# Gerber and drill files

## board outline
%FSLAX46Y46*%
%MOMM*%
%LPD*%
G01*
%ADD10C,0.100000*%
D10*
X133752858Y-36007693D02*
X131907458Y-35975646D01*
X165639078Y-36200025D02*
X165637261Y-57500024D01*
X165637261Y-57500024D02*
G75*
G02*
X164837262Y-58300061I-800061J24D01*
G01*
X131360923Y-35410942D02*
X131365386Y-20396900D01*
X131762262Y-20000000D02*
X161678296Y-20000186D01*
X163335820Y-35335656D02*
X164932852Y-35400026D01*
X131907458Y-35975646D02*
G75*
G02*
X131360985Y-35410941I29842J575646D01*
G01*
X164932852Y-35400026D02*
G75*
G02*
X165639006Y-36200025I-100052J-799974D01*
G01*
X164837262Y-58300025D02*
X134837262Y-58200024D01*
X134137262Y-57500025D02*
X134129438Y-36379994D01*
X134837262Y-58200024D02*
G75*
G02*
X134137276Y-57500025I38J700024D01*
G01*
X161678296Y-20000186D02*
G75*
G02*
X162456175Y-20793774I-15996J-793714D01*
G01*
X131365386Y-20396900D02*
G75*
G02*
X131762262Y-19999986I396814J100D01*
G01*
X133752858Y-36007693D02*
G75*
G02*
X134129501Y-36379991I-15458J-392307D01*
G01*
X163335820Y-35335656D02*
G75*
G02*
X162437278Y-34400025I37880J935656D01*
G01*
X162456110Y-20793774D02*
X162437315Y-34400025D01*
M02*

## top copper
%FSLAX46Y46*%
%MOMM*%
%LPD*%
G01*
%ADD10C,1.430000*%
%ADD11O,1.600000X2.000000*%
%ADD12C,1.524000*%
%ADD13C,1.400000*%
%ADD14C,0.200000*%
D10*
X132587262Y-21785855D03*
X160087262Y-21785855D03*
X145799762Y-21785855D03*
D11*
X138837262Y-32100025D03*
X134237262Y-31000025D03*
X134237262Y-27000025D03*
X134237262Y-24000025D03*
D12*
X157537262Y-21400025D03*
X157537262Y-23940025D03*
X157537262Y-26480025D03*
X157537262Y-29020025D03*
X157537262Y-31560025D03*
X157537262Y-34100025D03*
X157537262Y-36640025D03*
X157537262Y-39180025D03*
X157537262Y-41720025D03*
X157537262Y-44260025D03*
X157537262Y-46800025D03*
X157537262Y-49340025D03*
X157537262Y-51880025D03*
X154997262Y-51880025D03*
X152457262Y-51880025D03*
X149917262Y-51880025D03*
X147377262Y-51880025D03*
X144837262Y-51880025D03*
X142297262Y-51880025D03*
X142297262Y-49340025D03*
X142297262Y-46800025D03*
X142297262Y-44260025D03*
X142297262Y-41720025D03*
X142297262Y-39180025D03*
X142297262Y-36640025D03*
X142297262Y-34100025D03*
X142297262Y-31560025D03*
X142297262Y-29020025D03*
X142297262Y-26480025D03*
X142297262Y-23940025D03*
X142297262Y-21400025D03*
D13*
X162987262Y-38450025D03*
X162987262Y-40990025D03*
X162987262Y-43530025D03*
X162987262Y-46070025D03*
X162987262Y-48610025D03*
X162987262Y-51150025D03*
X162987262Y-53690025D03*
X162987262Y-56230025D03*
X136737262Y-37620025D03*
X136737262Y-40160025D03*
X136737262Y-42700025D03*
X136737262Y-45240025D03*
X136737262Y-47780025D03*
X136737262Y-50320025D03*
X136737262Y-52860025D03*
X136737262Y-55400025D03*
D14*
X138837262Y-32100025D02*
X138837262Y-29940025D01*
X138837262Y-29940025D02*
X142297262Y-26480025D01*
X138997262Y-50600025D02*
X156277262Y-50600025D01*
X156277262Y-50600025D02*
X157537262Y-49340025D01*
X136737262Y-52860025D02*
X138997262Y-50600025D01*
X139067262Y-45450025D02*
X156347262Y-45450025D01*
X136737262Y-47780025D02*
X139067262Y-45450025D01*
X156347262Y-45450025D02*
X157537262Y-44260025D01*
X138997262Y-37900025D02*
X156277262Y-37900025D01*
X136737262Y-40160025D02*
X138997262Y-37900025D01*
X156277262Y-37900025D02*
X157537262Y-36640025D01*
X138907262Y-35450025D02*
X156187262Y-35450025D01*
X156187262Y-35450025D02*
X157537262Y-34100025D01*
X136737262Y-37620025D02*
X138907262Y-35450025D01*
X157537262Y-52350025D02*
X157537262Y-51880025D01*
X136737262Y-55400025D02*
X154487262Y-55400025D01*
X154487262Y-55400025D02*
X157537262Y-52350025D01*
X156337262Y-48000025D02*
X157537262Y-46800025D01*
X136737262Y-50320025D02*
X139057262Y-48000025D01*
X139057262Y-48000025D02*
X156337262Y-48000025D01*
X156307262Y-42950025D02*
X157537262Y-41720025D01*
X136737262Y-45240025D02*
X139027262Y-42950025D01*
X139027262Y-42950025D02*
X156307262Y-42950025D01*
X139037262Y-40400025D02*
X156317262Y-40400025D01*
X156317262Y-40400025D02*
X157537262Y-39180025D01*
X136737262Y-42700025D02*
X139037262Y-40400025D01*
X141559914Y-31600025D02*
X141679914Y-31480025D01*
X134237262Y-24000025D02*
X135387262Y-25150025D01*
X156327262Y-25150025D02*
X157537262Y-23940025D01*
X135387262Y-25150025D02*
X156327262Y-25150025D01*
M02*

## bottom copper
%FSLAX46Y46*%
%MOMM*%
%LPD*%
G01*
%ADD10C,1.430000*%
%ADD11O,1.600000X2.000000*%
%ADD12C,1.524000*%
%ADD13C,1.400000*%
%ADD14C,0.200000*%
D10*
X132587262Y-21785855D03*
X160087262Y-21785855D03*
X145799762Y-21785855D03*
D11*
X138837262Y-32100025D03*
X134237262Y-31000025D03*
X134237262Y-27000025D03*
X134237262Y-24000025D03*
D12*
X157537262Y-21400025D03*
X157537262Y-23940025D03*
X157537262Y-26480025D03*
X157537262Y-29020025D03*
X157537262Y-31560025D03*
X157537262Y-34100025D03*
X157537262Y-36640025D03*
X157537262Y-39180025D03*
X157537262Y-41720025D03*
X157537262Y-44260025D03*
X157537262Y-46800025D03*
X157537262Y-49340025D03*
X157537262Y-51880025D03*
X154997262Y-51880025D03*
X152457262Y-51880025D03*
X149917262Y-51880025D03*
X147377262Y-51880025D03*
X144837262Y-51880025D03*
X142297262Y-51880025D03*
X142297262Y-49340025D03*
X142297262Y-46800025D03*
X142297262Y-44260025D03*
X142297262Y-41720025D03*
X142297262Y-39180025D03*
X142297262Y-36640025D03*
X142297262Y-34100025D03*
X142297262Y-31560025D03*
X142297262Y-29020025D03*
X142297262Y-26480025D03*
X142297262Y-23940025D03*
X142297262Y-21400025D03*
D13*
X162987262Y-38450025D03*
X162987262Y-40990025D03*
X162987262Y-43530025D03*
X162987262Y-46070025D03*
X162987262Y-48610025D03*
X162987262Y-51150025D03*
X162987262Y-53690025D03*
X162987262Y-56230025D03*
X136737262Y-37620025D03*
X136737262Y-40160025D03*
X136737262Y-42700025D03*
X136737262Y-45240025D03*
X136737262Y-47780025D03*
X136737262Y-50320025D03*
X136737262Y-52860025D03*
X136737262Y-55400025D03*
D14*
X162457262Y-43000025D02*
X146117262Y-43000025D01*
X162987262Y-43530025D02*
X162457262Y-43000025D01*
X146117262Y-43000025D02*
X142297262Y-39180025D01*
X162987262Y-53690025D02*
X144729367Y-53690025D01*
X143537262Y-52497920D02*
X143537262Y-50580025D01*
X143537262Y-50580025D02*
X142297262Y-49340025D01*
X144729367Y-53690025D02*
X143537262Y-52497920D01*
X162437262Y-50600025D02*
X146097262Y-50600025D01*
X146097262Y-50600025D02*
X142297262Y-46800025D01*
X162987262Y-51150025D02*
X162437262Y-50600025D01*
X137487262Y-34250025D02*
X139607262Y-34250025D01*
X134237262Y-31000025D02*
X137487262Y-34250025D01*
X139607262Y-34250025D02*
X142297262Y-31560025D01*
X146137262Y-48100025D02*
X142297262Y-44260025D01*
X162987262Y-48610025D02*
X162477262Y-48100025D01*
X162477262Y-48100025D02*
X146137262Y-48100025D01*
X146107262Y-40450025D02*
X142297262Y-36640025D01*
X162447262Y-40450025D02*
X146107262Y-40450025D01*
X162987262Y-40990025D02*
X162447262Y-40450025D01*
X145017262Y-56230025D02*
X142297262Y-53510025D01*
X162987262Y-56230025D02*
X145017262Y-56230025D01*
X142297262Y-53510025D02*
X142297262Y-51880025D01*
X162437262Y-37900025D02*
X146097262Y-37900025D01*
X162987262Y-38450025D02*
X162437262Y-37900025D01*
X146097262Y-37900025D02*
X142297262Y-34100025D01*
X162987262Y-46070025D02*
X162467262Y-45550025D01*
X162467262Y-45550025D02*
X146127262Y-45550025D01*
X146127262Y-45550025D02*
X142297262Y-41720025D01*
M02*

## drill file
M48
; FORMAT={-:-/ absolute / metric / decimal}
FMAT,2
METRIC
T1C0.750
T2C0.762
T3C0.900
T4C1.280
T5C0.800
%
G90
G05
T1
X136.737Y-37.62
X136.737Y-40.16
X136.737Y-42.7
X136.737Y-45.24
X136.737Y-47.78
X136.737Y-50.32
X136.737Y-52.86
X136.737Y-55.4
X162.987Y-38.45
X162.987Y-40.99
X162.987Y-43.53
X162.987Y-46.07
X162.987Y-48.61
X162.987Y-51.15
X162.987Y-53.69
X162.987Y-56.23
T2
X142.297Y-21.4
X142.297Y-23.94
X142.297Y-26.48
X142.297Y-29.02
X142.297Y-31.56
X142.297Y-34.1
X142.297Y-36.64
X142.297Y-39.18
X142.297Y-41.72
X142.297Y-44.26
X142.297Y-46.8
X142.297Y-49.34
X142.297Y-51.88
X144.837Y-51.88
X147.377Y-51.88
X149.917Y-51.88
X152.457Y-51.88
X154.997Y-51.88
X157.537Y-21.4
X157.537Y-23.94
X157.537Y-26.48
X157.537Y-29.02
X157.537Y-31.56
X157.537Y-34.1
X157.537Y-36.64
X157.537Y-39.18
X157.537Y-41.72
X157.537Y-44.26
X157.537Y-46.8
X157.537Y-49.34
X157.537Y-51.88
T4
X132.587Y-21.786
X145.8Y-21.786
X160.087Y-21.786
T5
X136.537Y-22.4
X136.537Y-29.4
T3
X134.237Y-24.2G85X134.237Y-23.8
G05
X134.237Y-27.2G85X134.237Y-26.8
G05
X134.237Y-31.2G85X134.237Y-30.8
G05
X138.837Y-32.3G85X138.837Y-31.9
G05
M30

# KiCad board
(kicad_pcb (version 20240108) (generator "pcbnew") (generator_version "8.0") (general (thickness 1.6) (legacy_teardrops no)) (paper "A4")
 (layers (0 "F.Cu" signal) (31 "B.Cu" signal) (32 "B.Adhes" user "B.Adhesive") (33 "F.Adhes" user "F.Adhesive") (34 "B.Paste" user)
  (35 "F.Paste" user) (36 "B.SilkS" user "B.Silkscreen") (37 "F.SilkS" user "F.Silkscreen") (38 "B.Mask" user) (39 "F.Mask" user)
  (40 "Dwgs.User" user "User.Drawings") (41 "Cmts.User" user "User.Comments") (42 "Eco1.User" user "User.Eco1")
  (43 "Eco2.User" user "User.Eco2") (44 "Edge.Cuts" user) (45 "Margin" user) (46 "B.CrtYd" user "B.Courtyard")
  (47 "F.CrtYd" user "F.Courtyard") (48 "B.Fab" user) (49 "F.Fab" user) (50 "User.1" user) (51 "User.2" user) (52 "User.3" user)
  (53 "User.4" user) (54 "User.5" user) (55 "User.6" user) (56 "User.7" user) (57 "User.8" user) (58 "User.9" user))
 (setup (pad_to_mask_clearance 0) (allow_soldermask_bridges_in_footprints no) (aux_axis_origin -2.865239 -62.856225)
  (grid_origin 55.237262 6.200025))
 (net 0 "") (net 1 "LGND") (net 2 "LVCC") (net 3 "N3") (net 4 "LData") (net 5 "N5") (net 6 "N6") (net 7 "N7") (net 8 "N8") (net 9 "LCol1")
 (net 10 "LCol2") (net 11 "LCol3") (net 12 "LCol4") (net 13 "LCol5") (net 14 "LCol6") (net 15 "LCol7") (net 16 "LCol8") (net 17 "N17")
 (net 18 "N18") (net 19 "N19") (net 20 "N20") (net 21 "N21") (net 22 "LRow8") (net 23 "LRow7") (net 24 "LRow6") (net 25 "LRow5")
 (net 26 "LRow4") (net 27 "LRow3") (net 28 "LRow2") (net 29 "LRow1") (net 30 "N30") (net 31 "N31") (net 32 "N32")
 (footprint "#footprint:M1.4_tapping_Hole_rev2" (layer "F.Cu") (at 148.137262 23.700025 -90)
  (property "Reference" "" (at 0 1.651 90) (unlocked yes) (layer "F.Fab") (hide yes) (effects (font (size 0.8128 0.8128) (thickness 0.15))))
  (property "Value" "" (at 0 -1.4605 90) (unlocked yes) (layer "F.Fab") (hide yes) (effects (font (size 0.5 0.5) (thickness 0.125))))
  (pad "" thru_hole circle (at -1.91417 15.55 270) (size 1.43 1.43) (drill 1.28) (layers "*.Cu" "*.Mask") (remove_unused_layers no)))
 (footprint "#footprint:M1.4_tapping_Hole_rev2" (layer "F.Cu") (at 160.087262 21.785855 -90)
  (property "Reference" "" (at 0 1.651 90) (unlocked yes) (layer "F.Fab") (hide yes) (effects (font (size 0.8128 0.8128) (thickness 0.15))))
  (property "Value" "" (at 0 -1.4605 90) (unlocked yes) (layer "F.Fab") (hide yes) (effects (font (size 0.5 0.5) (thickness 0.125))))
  (pad "" thru_hole circle (at 0 0 270) (size 1.43 1.43) (drill 1.28) (layers "*.Cu" "*.Mask") (remove_unused_layers no)))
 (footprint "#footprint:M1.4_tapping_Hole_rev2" (layer "F.Cu") (at 145.799762 21.785855 -90)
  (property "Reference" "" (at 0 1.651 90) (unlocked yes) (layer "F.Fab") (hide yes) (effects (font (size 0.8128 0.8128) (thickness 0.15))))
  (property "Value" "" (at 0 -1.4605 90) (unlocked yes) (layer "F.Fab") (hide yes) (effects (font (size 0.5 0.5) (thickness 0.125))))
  (pad "" thru_hole circle (at 0 0 270) (size 1.43 1.43) (drill 1.28) (layers "*.Cu" "*.Mask") (remove_unused_layers no)))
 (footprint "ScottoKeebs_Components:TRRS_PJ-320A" (layer "B.Cu") (at 136.537262 20.800025 180)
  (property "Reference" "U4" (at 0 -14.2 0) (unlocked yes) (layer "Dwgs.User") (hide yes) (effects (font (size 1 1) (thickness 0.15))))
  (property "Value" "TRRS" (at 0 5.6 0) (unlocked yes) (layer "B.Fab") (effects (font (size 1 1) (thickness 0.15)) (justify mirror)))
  (pad "" np_thru_hole circle (at 0 -8.6 180) (size 0.8 0.8) (drill 0.8) (layers "*.Cu" "*.Mask"))
  (pad "" np_thru_hole circle (at 0 -1.6 180) (size 0.8 0.8) (drill 0.8) (layers "*.Cu" "*.Mask"))
  (pad "1" thru_hole oval (at -2.3 -11.3 180) (size 1.6 2) (drill oval 0.9 1.3) (layers "*.Cu" "*.Mask") (remove_unused_layers no)
   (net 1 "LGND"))
  (pad "2" thru_hole oval (at 2.3 -10.2 180) (size 1.6 2) (drill oval 0.9 1.3) (layers "*.Cu" "*.Mask") (remove_unused_layers no)
   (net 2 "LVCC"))
  (pad "3" thru_hole oval (at 2.3 -6.2 180) (size 1.6 2) (drill oval 0.9 1.3) (layers "*.Cu" "*.Mask") (remove_unused_layers no)
   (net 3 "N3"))
  (pad "4" thru_hole oval (at 2.3 -3.2 180) (size 1.6 2) (drill oval 0.9 1.3) (layers "*.Cu" "*.Mask") (remove_unused_layers no)
   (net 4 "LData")))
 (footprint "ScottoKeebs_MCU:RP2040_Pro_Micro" (layer "B.Cu") (at 149.917262 37.910025 180)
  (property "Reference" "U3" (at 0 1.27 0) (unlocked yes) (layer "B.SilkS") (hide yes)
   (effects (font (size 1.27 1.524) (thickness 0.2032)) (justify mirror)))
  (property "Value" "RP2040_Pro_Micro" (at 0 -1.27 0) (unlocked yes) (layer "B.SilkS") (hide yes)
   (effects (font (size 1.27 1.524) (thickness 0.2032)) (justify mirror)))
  (pad "1" thru_hole circle (at -7.62 16.51 180) (size 1.524 1.524) (drill 0.762) (layers "*.Cu" "*.Mask") (remove_unused_layers no)
   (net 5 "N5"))
  (pad "2" thru_hole circle (at -7.62 13.97 180) (size 1.524 1.524) (drill 0.762) (layers "*.Cu" "*.Mask") (remove_unused_layers no)
   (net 4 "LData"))
  (pad "3" thru_hole circle (at -7.62 11.43 180) (size 1.524 1.524) (drill 0.762) (layers "*.Cu" "*.Mask") (remove_unused_layers no)
   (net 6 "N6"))
  (pad "4" thru_hole circle (at -7.62 8.89 180) (size 1.524 1.524) (drill 0.762) (layers "*.Cu" "*.Mask") (remove_unused_layers no)
   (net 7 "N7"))
  (pad "5" thru_hole circle (at -7.62 6.35 180) (size 1.524 1.524) (drill 0.762) (layers "*.Cu" "*.Mask") (remove_unused_layers no)
   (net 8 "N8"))
  (pad "6" thru_hole circle (at -7.62 3.81 180) (size 1.524 1.524) (drill 0.762) (layers "*.Cu" "*.Mask") (remove_unused_layers no)
   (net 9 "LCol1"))
  (pad "7" thru_hole circle (at -7.62 1.27 180) (size 1.524 1.524) (drill 0.762) (layers "*.Cu" "*.Mask") (remove_unused_layers no)
   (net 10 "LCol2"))
  (pad "8" thru_hole circle (at -7.62 -1.27 180) (size 1.524 1.524) (drill 0.762) (layers "*.Cu" "*.Mask") (remove_unused_layers no)
   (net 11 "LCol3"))
  (pad "9" thru_hole circle (at -7.62 -3.81 180) (size 1.524 1.524) (drill 0.762) (layers "*.Cu" "*.Mask") (remove_unused_layers no)
   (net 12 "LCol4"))
  (pad "10" thru_hole circle (at -7.62 -6.35 180) (size 1.524 1.524) (drill 0.762) (layers "*.Cu" "*.Mask") (remove_unused_layers no)
   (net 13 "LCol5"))
  (pad "11" thru_hole circle (at -7.62 -8.89 180) (size 1.524 1.524) (drill 0.762) (layers "*.Cu" "*.Mask") (remove_unused_layers no)
   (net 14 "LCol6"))
  (pad "12" thru_hole circle (at -7.62 -11.43 180) (size 1.524 1.524) (drill 0.762) (layers "*.Cu" "*.Mask") (remove_unused_layers no)
   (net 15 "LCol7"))
  (pad "13" thru_hole circle (at -7.62 -13.97 180) (size 1.524 1.524) (drill 0.762) (layers "*.Cu" "*.Mask") (remove_unused_layers no)
   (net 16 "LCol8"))
  (pad "14" thru_hole circle (at -5.08 -13.97 180) (size 1.524 1.524) (drill 0.762) (layers "*.Cu" "*.Mask") (remove_unused_layers no)
   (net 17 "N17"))
  (pad "15" thru_hole circle (at -2.54 -13.97 180) (size 1.524 1.524) (drill 0.762) (layers "*.Cu" "*.Mask") (remove_unused_layers no)
   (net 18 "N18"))
  (pad "16" thru_hole circle (at 0 -13.97 180) (size 1.524 1.524) (drill 0.762) (layers "*.Cu" "*.Mask") (remove_unused_layers no)
   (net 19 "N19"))
  (pad "17" thru_hole circle (at 2.54 -13.97 180) (size 1.524 1.524) (drill 0.762) (layers "*.Cu" "*.Mask") (remove_unused_layers no)
   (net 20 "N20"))
  (pad "18" thru_hole circle (at 5.08 -13.97 180) (size 1.524 1.524) (drill 0.762) (layers "*.Cu" "*.Mask") (remove_unused_layers no)
   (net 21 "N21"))
  (pad "19" thru_hole circle (at 7.62 -13.97 180) (size 1.524 1.524) (drill 0.762) (layers "*.Cu" "*.Mask") (remove_unused_layers no)
   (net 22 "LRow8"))
  (pad "20" thru_hole circle (at 7.62 -11.43 180) (size 1.524 1.524) (drill 0.762) (layers "*.Cu" "*.Mask") (remove_unused_layers no)
   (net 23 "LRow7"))
  (pad "21" thru_hole circle (at 7.62 -8.89 180) (size 1.524 1.524) (drill 0.762) (layers "*.Cu" "*.Mask") (remove_unused_layers no)
   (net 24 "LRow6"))
  (pad "22" thru_hole circle (at 7.62 -6.35 180) (size 1.524 1.524) (drill 0.762) (layers "*.Cu" "*.Mask") (remove_unused_layers no)
   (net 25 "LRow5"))
  (pad "23" thru_hole circle (at 7.62 -3.81 180) (size 1.524 1.524) (drill 0.762) (layers "*.Cu" "*.Mask") (remove_unused_layers no)
   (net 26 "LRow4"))
  (pad "24" thru_hole circle (at 7.62 -1.27 180) (size 1.524 1.524) (drill 0.762) (layers "*.Cu" "*.Mask") (remove_unused_layers no)
   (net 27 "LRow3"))
  (pad "25" thru_hole circle (at 7.62 1.27 180) (size 1.524 1.524) (drill 0.762) (layers "*.Cu" "*.Mask") (remove_unused_layers no)
   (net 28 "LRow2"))
  (pad "26" thru_hole circle (at 7.62 3.81 180) (size 1.524 1.524) (drill 0.762) (layers "*.Cu" "*.Mask") (remove_unused_layers no)
   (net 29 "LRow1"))
  (pad "27" thru_hole circle (at 7.62 6.35 180) (size 1.524 1.524) (drill 0.762) (layers "*.Cu" "*.Mask") (remove_unused_layers no)
   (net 2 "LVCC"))
  (pad "28" thru_hole circle (at 7.62 8.89 180) (size 1.524 1.524) (drill 0.762) (layers "*.Cu" "*.Mask") (remove_unused_layers no)
   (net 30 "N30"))
  (pad "29" thru_hole circle (at 7.62 11.43 180) (size 1.524 1.524) (drill 0.762) (layers "*.Cu" "*.Mask") (remove_unused_layers no)
   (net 1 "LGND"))
  (pad "30" thru_hole circle (at 7.62 13.97 180) (size 1.524 1.524) (drill 0.762) (layers "*.Cu" "*.Mask") (remove_unused_layers no)
   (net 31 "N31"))
  (pad "31" thru_hole circle (at 7.62 16.51 180) (size 1.524 1.524) (drill 0.762) (layers "*.Cu" "*.Mask") (remove_unused_layers no)
   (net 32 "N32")))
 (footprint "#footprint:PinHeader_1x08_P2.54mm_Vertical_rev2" (layer "B.Cu") (at 162.987262 38.450025 180)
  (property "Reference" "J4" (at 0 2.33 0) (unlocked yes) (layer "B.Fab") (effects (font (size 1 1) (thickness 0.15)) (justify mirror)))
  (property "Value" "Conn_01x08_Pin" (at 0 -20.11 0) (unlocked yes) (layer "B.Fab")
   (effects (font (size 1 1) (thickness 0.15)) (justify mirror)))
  (pad "1" thru_hole circle (at 0 0 180) (size 1.4 1.4) (drill 0.75) (layers "*.Cu" "*.Mask") (remove_unused_layers no) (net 29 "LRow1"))
  (pad "2" thru_hole circle (at 0 -2.54 180) (size 1.4 1.4) (drill 0.75) (layers "*.Cu" "*.Mask") (remove_unused_layers no) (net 28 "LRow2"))
  (pad "3" thru_hole circle (at 0 -5.08 180) (size 1.4 1.4) (drill 0.75) (layers "*.Cu" "*.Mask") (remove_unused_layers no) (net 27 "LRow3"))
  (pad "4" thru_hole circle (at 0 -7.62 180) (size 1.4 1.4) (drill 0.75) (layers "*.Cu" "*.Mask") (remove_unused_layers no) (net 26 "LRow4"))
  (pad "5" thru_hole circle (at 0 -10.16 180) (size 1.4 1.4) (drill 0.75) (layers "*.Cu" "*.Mask") (remove_unused_layers no)
   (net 25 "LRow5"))
  (pad "6" thru_hole circle (at 0 -12.7 180) (size 1.4 1.4) (drill 0.75) (layers "*.Cu" "*.Mask") (remove_unused_layers no) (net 24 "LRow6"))
  (pad "7" thru_hole circle (at 0 -15.24 180) (size 1.4 1.4) (drill 0.75) (layers "*.Cu" "*.Mask") (remove_unused_layers no)
   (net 23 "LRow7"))
  (pad "8" thru_hole circle (at 0 -17.78 180) (size 1.4 1.4) (drill 0.75) (layers "*.Cu" "*.Mask") (remove_unused_layers no)
   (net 22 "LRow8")))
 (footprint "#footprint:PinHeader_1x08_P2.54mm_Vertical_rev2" (layer "B.Cu") (at 136.737262 37.620025 180)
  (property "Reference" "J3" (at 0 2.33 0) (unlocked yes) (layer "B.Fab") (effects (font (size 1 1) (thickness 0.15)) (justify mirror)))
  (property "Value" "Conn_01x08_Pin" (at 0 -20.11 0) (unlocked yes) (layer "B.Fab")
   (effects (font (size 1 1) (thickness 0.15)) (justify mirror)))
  (pad "1" thru_hole circle (at 0 0 180) (size 1.4 1.4) (drill 0.75) (layers "*.Cu" "*.Mask") (remove_unused_layers no) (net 9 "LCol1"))
  (pad "2" thru_hole circle (at 0 -2.54 180) (size 1.4 1.4) (drill 0.75) (layers "*.Cu" "*.Mask") (remove_unused_layers no) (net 10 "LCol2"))
  (pad "3" thru_hole circle (at 0 -5.08 180) (size 1.4 1.4) (drill 0.75) (layers "*.Cu" "*.Mask") (remove_unused_layers no) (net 11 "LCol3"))
  (pad "4" thru_hole circle (at 0 -7.62 180) (size 1.4 1.4) (drill 0.75) (layers "*.Cu" "*.Mask") (remove_unused_layers no) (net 12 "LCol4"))
  (pad "5" thru_hole circle (at 0 -10.16 180) (size 1.4 1.4) (drill 0.75) (layers "*.Cu" "*.Mask") (remove_unused_layers no)
   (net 13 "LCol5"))
  (pad "6" thru_hole circle (at 0 -12.7 180) (size 1.4 1.4) (drill 0.75) (layers "*.Cu" "*.Mask") (remove_unused_layers no) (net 14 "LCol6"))
  (pad "7" thru_hole circle (at 0 -15.24 180) (size 1.4 1.4) (drill 0.75) (layers "*.Cu" "*.Mask") (remove_unused_layers no)
   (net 15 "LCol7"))
  (pad "8" thru_hole circle (at 0 -17.78 180) (size 1.4 1.4) (drill 0.75) (layers "*.Cu" "*.Mask") (remove_unused_layers no)
   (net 16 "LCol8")))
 (gr_line (start 133.752858 36.007693) (end 131.907458 35.975646) (stroke (width 0.1) (type default)) (layer "Edge.Cuts"))
 (gr_line (start 165.639078 36.200025) (end 165.637261 57.500024) (stroke (width 0.1) (type default)) (layer "Edge.Cuts"))
 (gr_arc (start 165.637261 57.500024) (mid 165.402937 58.0657) (end 164.837262 58.300025) (stroke (width 0.1) (type default))
  (layer "Edge.Cuts"))
 (gr_line (start 131.360923 35.410942) (end 131.365386 20.3969) (stroke (width 0.1) (type default)) (layer "Edge.Cuts"))
 (gr_line (start 131.762262 20) (end 161.678296 20.000186) (stroke (width 0.1) (type default)) (layer "Edge.Cuts"))
 (gr_line (start 163.33582 35.335656) (end 164.932852 35.400026) (stroke (width 0.1) (type default)) (layer "Edge.Cuts"))
 (gr_arc (start 131.907458 35.975646) (mid 131.523045 35.800863) (end 131.360923 35.410942) (stroke (width 0.1) (type default))
  (layer "Edge.Cuts"))
 (gr_arc (start 164.932852 35.400026) (mid 165.437261 35.666464) (end 165.639078 36.200025) (stroke (width 0.1) (type default))
  (layer "Edge.Cuts"))
 (gr_line (start 164.837262 58.300025) (end 134.837262 58.200024) (stroke (width 0.1) (type default)) (layer "Edge.Cuts"))
 (gr_line (start 134.137262 57.500025) (end 134.129438 36.379994) (stroke (width 0.1) (type default)) (layer "Edge.Cuts"))
 (gr_arc (start 134.837262 58.200024) (mid 134.342285 57.995001) (end 134.137262 57.500025) (stroke (width 0.1) (type default))
  (layer "Edge.Cuts"))
 (gr_arc (start 161.678296 20.000186) (mid 162.229203 20.2382) (end 162.45611 20.793774) (stroke (width 0.1) (type default))
  (layer "Edge.Cuts"))
 (gr_arc (start 131.365386 20.3969) (mid 131.481589 20.116221) (end 131.762262 20) (stroke (width 0.1) (type default)) (layer "Edge.Cuts"))
 (gr_arc (start 133.752858 36.007693) (mid 134.013376 36.120802) (end 134.129438 36.379994) (stroke (width 0.1) (type default))
  (layer "Edge.Cuts"))
 (gr_arc (start 163.33582 35.335656) (mid 162.698334 35.048622) (end 162.437315 34.400025) (stroke (width 0.1) (type default))
  (layer "Edge.Cuts"))
 (gr_line (start 162.45611 20.793774) (end 162.437315 34.400025) (stroke (width 0.1) (type default)) (layer "Edge.Cuts"))
 (segment (start 138.837262 32.100025) (end 138.837262 29.940025) (width 0.2) (layer "F.Cu") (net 1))
 (segment (start 138.837262 29.940025) (end 142.297262 26.480025) (width 0.2) (layer "F.Cu") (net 1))
 (segment (start 138.997262 50.600025) (end 156.277262 50.600025) (width 0.2) (layer "F.Cu") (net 15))
 (segment (start 156.277262 50.600025) (end 157.537262 49.340025) (width 0.2) (layer "F.Cu") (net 15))
 (segment (start 136.737262 52.860025) (end 138.997262 50.600025) (width 0.2) (layer "F.Cu") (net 15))
 (segment (start 139.067262 45.450025) (end 156.347262 45.450025) (width 0.2) (layer "F.Cu") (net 13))
 (segment (start 136.737262 47.780025) (end 139.067262 45.450025) (width 0.2) (layer "F.Cu") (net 13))
 (segment (start 156.347262 45.450025) (end 157.537262 44.260025) (width 0.2) (layer "F.Cu") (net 13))
 (segment (start 138.997262 37.900025) (end 156.277262 37.900025) (width 0.2) (layer "F.Cu") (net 10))
 (segment (start 136.737262 40.160025) (end 138.997262 37.900025) (width 0.2) (layer "F.Cu") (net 10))
 (segment (start 156.277262 37.900025) (end 157.537262 36.640025) (width 0.2) (layer "F.Cu") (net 10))
 (segment (start 138.907262 35.450025) (end 156.187262 35.450025) (width 0.2) (layer "F.Cu") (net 9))
 (segment (start 156.187262 35.450025) (end 157.537262 34.100025) (width 0.2) (layer "F.Cu") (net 9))
 (segment (start 136.737262 37.620025) (end 138.907262 35.450025) (width 0.2) (layer "F.Cu") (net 9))
 (segment (start 157.537262 52.350025) (end 157.537262 51.880025) (width 0.2) (layer "F.Cu") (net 16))
 (segment (start 136.737262 55.400025) (end 154.487262 55.400025) (width 0.2) (layer "F.Cu") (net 16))
 (segment (start 154.487262 55.400025) (end 157.537262 52.350025) (width 0.2) (layer "F.Cu") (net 16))
 (segment (start 156.337262 48.000025) (end 157.537262 46.800025) (width 0.2) (layer "F.Cu") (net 14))
 (segment (start 136.737262 50.320025) (end 139.057262 48.000025) (width 0.2) (layer "F.Cu") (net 14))
 (segment (start 139.057262 48.000025) (end 156.337262 48.000025) (width 0.2) (layer "F.Cu") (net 14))
 (segment (start 156.307262 42.950025) (end 157.537262 41.720025) (width 0.2) (layer "F.Cu") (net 12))
 (segment (start 136.737262 45.240025) (end 139.027262 42.950025) (width 0.2) (layer "F.Cu") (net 12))
 (segment (start 139.027262 42.950025) (end 156.307262 42.950025) (width 0.2) (layer "F.Cu") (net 12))
 (segment (start 139.037262 40.400025) (end 156.317262 40.400025) (width 0.2) (layer "F.Cu") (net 11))
 (segment (start 156.317262 40.400025) (end 157.537262 39.180025) (width 0.2) (layer "F.Cu") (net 11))
 (segment (start 136.737262 42.700025) (end 139.037262 40.400025) (width 0.2) (layer "F.Cu") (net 11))
 (segment (start 162.457262 43.000025) (end 146.117262 43.000025) (width 0.2) (layer "B.Cu") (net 27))
 (segment (start 162.987262 43.530025) (end 162.457262 43.000025) (width 0.2) (layer "B.Cu") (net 27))
 (segment (start 146.117262 43.000025) (end 142.297262 39.180025) (width 0.2) (layer "B.Cu") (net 27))
 (segment (start 162.987262 53.690025) (end 144.729367 53.690025) (width 0.2) (layer "B.Cu") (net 23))
 (segment (start 143.537262 52.49792) (end 143.537262 50.580025) (width 0.2) (layer "B.Cu") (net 23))
 (segment (start 143.537262 50.580025) (end 142.297262 49.340025) (width 0.2) (layer "B.Cu") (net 23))
 (segment (start 144.729367 53.690025) (end 143.537262 52.49792) (width 0.2) (layer "B.Cu") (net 23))
 (segment (start 162.437262 50.600025) (end 146.097262 50.600025) (width 0.2) (layer "B.Cu") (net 24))
 (segment (start 146.097262 50.600025) (end 142.297262 46.800025) (width 0.2) (layer "B.Cu") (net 24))
 (segment (start 162.987262 51.150025) (end 162.437262 50.600025) (width 0.2) (layer "B.Cu") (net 24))
 (segment (start 141.559914 31.600025) (end 141.679914 31.480025) (width 0.2) (layer "F.Cu") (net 2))
 (segment (start 137.487262 34.250025) (end 139.607262 34.250025) (width 0.2) (layer "B.Cu") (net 2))
 (segment (start 134.237262 31.000025) (end 137.487262 34.250025) (width 0.2) (layer "B.Cu") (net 2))
 (segment (start 139.607262 34.250025) (end 142.297262 31.560025) (width 0.2) (layer "B.Cu") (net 2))
 (segment (start 134.237262 24.000025) (end 135.387262 25.150025) (width 0.2) (layer "F.Cu") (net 4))
 (segment (start 156.327262 25.150025) (end 157.537262 23.940025) (width 0.2) (layer "F.Cu") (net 4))
 (segment (start 135.387262 25.150025) (end 156.327262 25.150025) (width 0.2) (layer "F.Cu") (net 4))
 (segment (start 146.137262 48.100025) (end 142.297262 44.260025) (width 0.2) (layer "B.Cu") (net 25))
 (segment (start 162.987262 48.610025) (end 162.477262 48.100025) (width 0.2) (layer "B.Cu") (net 25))
 (segment (start 162.477262 48.100025) (end 146.137262 48.100025) (width 0.2) (layer "B.Cu") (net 25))
 (segment (start 146.107262 40.450025) (end 142.297262 36.640025) (width 0.2) (layer "B.Cu") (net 28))
 (segment (start 162.447262 40.450025) (end 146.107262 40.450025) (width 0.2) (layer "B.Cu") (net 28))
 (segment (start 162.987262 40.990025) (end 162.447262 40.450025) (width 0.2) (layer "B.Cu") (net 28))
 (segment (start 145.017262 56.230025) (end 142.297262 53.510025) (width 0.2) (layer "B.Cu") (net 22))
 (segment (start 162.987262 56.230025) (end 145.017262 56.230025) (width 0.2) (layer "B.Cu") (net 22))
 (segment (start 142.297262 53.510025) (end 142.297262 51.880025) (width 0.2) (layer "B.Cu") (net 22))
 (segment (start 162.437262 37.900025) (end 146.097262 37.900025) (width 0.2) (layer "B.Cu") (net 29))
 (segment (start 162.987262 38.450025) (end 162.437262 37.900025) (width 0.2) (layer "B.Cu") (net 29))
 (segment (start 146.097262 37.900025) (end 142.297262 34.100025) (width 0.2) (layer "B.Cu") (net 29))
 (segment (start 162.987262 46.070025) (end 162.467262 45.550025) (width 0.2) (layer "B.Cu") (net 26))
 (segment (start 162.467262 45.550025) (end 146.127262 45.550025) (width 0.2) (layer "B.Cu") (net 26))
 (segment (start 146.127262 45.550025) (end 142.297262 41.720025) (width 0.2) (layer "B.Cu") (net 26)))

